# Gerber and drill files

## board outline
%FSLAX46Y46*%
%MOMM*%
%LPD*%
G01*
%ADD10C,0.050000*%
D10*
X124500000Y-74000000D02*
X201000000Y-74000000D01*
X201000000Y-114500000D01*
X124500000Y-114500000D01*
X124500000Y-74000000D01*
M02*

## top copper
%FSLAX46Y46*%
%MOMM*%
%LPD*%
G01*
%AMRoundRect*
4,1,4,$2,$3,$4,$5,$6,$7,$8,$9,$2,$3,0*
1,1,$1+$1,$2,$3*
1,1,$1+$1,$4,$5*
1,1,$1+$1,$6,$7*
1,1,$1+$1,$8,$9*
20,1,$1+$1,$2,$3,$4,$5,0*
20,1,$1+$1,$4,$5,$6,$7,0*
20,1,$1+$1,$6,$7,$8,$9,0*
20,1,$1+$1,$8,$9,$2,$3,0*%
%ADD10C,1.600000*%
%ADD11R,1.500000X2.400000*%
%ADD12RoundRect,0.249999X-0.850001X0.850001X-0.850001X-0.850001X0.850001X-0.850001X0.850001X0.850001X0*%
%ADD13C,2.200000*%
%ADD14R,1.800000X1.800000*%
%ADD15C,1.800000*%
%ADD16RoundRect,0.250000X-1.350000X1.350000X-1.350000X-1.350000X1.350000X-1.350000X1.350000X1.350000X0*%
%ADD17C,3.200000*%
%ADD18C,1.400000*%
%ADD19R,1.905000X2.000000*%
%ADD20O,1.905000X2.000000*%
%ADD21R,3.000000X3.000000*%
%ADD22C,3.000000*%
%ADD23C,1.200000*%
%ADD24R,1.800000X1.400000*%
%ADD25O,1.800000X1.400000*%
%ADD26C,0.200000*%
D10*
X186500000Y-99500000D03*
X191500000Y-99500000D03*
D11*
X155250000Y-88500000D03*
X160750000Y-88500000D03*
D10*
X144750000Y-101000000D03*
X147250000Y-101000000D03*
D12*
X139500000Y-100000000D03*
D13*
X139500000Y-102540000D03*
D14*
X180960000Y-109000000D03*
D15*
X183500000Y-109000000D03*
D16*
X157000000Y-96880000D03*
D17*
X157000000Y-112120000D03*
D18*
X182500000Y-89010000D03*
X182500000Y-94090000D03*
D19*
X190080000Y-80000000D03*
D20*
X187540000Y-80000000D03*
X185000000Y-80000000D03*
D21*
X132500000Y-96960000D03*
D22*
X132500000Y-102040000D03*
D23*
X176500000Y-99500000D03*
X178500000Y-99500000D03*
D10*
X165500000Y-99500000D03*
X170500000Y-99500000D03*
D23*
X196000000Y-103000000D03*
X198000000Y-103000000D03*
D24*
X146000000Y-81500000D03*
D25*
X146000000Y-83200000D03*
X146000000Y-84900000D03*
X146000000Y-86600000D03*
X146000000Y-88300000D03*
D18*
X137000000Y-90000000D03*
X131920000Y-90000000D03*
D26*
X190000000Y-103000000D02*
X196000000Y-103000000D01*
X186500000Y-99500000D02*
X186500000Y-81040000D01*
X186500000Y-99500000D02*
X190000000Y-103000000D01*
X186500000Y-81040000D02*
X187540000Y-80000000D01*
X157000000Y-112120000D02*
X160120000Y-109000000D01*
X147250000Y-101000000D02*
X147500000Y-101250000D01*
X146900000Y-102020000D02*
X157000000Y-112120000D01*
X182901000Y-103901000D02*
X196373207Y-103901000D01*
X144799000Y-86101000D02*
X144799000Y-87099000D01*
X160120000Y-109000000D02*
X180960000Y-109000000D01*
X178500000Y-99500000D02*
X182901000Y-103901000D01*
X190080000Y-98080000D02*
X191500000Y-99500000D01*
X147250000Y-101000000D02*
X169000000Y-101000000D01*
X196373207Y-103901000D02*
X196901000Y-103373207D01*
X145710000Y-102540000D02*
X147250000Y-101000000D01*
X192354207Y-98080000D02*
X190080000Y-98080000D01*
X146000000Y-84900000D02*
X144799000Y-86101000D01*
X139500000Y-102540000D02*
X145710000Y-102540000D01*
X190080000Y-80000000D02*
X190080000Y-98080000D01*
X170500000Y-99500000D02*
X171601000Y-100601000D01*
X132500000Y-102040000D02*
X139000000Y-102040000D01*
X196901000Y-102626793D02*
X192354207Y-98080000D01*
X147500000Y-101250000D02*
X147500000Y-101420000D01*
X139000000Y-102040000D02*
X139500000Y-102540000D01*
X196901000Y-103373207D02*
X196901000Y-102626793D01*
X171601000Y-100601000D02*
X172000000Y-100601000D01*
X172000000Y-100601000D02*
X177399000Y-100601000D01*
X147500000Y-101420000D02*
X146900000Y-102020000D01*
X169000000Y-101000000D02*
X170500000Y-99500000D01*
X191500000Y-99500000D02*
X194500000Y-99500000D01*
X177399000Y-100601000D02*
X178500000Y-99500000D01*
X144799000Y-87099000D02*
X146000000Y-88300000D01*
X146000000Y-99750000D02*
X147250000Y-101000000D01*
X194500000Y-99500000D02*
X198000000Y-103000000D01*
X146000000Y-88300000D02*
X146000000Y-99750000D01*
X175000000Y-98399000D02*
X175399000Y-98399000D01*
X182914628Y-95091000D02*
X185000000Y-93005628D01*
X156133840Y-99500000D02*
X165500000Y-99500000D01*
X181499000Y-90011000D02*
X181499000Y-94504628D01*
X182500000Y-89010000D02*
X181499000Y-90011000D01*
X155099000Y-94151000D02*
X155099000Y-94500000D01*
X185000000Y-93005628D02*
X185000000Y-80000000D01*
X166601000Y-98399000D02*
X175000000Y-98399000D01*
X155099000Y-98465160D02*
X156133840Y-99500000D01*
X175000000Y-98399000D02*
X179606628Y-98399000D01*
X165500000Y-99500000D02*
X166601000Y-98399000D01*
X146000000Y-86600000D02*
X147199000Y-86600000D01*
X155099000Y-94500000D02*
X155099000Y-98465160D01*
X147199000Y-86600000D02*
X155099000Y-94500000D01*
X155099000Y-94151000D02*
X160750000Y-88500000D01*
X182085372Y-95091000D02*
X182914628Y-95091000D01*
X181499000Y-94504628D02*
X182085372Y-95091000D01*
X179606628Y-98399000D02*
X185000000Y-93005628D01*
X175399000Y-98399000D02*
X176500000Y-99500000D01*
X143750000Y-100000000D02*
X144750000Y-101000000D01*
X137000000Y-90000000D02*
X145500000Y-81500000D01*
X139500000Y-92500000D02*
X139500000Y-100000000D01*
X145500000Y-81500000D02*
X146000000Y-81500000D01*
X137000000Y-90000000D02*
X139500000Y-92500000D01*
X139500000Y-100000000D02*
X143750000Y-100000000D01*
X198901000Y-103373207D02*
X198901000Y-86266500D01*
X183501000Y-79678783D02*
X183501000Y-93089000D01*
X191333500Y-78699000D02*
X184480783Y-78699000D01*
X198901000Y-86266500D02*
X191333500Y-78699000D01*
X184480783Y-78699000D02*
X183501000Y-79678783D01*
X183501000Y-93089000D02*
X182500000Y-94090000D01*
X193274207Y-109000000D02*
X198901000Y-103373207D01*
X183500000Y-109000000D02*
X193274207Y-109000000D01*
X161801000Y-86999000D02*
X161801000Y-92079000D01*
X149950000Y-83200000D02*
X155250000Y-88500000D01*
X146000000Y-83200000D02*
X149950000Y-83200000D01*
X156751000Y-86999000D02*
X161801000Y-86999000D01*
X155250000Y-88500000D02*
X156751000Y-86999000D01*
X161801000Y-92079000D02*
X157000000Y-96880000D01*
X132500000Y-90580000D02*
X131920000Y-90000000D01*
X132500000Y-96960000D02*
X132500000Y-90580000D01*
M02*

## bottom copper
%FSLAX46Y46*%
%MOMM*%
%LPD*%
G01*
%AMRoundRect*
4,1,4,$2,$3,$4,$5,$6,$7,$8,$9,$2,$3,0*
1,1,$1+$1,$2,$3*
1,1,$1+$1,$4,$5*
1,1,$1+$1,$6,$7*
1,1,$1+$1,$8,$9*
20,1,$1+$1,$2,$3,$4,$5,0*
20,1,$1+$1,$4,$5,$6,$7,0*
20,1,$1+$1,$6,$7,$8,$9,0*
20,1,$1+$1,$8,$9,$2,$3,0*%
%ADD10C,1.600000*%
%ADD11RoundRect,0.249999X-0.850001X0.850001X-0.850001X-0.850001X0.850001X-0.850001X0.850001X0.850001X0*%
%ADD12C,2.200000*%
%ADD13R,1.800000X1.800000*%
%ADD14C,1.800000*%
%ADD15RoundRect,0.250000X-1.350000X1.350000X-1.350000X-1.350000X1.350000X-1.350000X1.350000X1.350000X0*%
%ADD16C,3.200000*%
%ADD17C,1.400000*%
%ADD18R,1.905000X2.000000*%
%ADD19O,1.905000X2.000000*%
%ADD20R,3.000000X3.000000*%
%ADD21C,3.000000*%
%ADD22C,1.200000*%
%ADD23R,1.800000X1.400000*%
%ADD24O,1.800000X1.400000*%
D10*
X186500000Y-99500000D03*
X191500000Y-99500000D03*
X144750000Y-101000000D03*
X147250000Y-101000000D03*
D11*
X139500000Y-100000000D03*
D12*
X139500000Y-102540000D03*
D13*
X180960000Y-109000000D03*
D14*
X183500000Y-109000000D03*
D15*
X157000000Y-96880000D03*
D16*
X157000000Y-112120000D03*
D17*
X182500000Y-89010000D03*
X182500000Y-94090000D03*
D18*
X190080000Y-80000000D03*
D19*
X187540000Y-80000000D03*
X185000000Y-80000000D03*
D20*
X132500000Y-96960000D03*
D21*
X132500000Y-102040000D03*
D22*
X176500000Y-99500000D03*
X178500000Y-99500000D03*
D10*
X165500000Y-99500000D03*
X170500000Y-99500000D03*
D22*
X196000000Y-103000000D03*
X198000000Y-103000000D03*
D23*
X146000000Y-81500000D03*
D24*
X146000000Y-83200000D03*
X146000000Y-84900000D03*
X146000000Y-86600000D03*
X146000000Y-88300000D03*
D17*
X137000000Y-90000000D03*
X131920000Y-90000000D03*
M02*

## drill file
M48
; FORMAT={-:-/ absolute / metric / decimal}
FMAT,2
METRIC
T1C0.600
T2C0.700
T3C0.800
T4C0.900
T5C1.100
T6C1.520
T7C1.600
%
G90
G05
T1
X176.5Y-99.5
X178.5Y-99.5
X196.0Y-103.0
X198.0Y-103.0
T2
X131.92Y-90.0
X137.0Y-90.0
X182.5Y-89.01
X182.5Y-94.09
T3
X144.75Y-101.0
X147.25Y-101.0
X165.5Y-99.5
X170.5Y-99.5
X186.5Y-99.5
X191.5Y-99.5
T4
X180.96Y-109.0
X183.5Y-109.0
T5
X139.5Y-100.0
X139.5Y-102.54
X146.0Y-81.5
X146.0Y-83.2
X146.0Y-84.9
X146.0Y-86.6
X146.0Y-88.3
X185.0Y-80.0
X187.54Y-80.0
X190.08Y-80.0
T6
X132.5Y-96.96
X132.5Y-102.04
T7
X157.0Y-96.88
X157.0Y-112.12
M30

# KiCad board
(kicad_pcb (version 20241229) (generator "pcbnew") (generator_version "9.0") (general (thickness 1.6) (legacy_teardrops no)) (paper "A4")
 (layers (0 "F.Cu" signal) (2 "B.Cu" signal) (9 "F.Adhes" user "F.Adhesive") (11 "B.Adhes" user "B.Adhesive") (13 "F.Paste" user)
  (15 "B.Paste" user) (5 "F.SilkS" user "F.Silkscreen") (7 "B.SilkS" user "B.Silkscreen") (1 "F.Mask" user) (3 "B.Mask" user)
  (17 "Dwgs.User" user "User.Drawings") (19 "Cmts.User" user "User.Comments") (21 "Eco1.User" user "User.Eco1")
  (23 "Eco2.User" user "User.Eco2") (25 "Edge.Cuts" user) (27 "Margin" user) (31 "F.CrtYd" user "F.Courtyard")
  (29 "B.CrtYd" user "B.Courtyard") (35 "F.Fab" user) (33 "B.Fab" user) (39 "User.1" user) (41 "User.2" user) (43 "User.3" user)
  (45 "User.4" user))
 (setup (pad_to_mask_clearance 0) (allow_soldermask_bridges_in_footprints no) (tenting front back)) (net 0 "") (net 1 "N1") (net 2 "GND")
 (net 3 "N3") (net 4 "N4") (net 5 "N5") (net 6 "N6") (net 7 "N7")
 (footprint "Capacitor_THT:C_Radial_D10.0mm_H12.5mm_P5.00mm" (layer "F.Cu") (at 186.5 99.5)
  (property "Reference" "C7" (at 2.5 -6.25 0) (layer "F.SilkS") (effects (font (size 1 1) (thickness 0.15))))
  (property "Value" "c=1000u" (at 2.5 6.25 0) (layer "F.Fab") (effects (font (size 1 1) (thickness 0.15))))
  (pad "1" thru_hole circle (at 0 0) (size 1.6 1.6) (drill 0.8) (layers "*.Cu" "*.Mask") (remove_unused_layers no) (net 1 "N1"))
  (pad "2" thru_hole circle (at 5 0) (size 1.6 1.6) (drill 0.8) (layers "*.Cu" "*.Mask") (remove_unused_layers no) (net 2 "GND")))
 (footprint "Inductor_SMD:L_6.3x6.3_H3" (layer "F.Cu") (at 158 88.5)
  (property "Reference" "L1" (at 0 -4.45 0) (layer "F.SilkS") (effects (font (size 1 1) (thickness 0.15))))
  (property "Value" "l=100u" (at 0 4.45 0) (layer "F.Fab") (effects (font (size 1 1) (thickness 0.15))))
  (pad "1" smd rect (at -2.75 0) (size 1.5 2.4) (layers "F.Cu" "F.Mask" "F.Paste") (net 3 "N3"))
  (pad "2" smd rect (at 2.75 0) (size 1.5 2.4) (layers "F.Cu" "F.Mask" "F.Paste") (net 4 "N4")))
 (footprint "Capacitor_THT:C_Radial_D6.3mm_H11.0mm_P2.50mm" (layer "F.Cu") (at 144.75 101)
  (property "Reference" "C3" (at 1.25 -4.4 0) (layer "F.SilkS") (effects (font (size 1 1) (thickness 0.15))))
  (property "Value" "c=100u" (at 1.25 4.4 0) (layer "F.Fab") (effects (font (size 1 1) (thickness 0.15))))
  (pad "1" thru_hole circle (at 0 0) (size 1.6 1.6) (drill 0.8) (layers "*.Cu" "*.Mask") (remove_unused_layers no) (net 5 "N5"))
  (pad "2" thru_hole circle (at 2.5 0) (size 1.6 1.6) (drill 0.8) (layers "*.Cu" "*.Mask") (remove_unused_layers no) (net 2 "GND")))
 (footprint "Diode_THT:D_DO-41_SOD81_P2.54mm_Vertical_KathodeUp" (layer "F.Cu") (at 139.5 100 -90)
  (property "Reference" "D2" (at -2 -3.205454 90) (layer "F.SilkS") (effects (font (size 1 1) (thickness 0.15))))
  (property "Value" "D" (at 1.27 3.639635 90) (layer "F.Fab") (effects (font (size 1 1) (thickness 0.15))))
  (pad "1" thru_hole roundrect (at 0 0 270) (size 2.2 2.2) (drill 1.1) (layers "*.Cu" "*.Mask") (remove_unused_layers no)
   (roundrect_rratio 0.113636) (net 5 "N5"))
  (pad "2" thru_hole circle (at 2.54 0 270) (size 2.2 2.2) (drill 1.1) (layers "*.Cu" "*.Mask") (remove_unused_layers no) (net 2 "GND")))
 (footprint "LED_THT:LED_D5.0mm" (layer "F.Cu") (at 180.96 109)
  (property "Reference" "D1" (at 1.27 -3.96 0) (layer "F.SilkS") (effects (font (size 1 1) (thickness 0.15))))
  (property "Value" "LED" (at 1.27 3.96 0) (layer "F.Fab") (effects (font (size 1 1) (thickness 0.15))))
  (pad "1" thru_hole rect (at 0 0) (size 1.8 1.8) (drill 0.9) (layers "*.Cu" "*.Mask") (remove_unused_layers no) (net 2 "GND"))
  (pad "2" thru_hole circle (at 2.54 0) (size 1.8 1.8) (drill 0.9) (layers "*.Cu" "*.Mask") (remove_unused_layers no) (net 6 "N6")))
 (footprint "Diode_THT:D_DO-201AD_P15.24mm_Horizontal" (layer "F.Cu") (at 157 96.88 -90)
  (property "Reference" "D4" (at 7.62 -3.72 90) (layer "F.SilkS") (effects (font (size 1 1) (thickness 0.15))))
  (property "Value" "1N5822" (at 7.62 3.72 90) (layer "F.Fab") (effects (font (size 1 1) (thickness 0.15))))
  (pad "1" thru_hole roundrect (at 0 0 270) (size 3.2 3.2) (drill 1.6) (layers "*.Cu" "*.Mask") (remove_unused_layers no)
   (roundrect_rratio 0.078125) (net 3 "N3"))
  (pad "2" thru_hole circle (at 15.24 0 270) (size 3.2 3.2) (drill 1.6) (layers "*.Cu" "*.Mask") (remove_unused_layers no) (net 2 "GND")))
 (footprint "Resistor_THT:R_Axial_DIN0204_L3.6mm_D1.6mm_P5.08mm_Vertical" (layer "F.Cu") (at 182.5 89.01 -90)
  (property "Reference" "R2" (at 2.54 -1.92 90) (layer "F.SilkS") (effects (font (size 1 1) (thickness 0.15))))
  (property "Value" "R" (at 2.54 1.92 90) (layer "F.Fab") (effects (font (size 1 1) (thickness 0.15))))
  (pad "1" thru_hole circle (at 0 0 270) (size 1.4 1.4) (drill 0.7) (layers "*.Cu" "*.Mask") (remove_unused_layers no) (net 4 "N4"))
  (pad "2" thru_hole circle (at 5.08 0 270) (size 1.4 1.4) (drill 0.7) (layers "*.Cu" "*.Mask") (remove_unused_layers no) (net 6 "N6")))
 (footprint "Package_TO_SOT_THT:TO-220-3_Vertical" (layer "F.Cu") (at 190.08 80 180)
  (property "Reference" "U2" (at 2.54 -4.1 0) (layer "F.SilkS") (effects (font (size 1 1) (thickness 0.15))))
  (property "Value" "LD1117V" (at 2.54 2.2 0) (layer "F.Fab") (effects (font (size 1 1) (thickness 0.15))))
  (pad "1" thru_hole rect (at 0 0 180) (size 1.905 2) (drill 1.1) (layers "*.Cu" "*.Mask") (remove_unused_layers no) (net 2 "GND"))
  (pad "2" thru_hole oval (at 2.54 0 180) (size 1.905 2) (drill 1.1) (layers "*.Cu" "*.Mask") (remove_unused_layers no) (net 1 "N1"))
  (pad "3" thru_hole oval (at 5.08 0 180) (size 1.905 2) (drill 1.1) (layers "*.Cu" "*.Mask") (remove_unused_layers no) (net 4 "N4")))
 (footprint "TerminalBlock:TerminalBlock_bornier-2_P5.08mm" (layer "F.Cu") (at 132.5 96.96 -90)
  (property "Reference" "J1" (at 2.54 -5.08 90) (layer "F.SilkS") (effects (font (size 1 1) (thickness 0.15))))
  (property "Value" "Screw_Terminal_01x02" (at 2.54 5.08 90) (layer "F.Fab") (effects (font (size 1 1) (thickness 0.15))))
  (pad "1" thru_hole rect (at 0 0 270) (size 3 3) (drill 1.52) (layers "*.Cu" "*.Mask") (remove_unused_layers no) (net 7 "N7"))
  (pad "2" thru_hole circle (at 5.08 0 270) (size 3 3) (drill 1.52) (layers "*.Cu" "*.Mask") (remove_unused_layers no) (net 2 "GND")))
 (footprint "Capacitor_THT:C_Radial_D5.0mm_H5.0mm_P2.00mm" (layer "F.Cu") (at 176.5 99.5)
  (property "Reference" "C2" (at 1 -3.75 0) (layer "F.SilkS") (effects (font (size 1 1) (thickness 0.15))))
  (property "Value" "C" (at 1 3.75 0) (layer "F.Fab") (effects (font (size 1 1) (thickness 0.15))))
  (pad "1" thru_hole circle (at 0 0) (size 1.2 1.2) (drill 0.6) (layers "*.Cu" "*.Mask") (remove_unused_layers no) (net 4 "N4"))
  (pad "2" thru_hole circle (at 2 0) (size 1.2 1.2) (drill 0.6) (layers "*.Cu" "*.Mask") (remove_unused_layers no) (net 2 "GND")))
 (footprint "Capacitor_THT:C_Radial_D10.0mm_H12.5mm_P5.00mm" (layer "F.Cu") (at 165.5 99.5)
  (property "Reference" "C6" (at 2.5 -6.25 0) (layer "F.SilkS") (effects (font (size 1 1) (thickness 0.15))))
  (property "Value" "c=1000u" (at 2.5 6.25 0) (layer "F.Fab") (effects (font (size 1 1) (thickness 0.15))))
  (pad "1" thru_hole circle (at 0 0) (size 1.6 1.6) (drill 0.8) (layers "*.Cu" "*.Mask") (remove_unused_layers no) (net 4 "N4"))
  (pad "2" thru_hole circle (at 5 0) (size 1.6 1.6) (drill 0.8) (layers "*.Cu" "*.Mask") (remove_unused_layers no) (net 2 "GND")))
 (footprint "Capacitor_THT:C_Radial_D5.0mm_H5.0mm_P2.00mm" (layer "F.Cu") (at 196 103)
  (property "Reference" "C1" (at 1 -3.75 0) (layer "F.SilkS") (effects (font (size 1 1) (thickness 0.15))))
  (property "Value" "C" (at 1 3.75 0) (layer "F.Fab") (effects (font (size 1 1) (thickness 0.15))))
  (pad "1" thru_hole circle (at 0 0) (size 1.2 1.2) (drill 0.6) (layers "*.Cu" "*.Mask") (remove_unused_layers no) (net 1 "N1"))
  (pad "2" thru_hole circle (at 2 0) (size 1.2 1.2) (drill 0.6) (layers "*.Cu" "*.Mask") (remove_unused_layers no) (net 2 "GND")))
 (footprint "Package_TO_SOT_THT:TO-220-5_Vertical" (layer "F.Cu") (at 146 81.5 -90)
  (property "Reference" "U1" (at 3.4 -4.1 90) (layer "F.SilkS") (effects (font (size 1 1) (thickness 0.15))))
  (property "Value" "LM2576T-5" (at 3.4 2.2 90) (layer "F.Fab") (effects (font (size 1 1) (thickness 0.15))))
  (pad "1" thru_hole rect (at 0 0 270) (size 1.4 1.8) (drill 1.1) (layers "*.Cu" "*.Mask") (remove_unused_layers no) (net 5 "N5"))
  (pad "2" thru_hole oval (at 1.7 0 270) (size 1.4 1.8) (drill 1.1) (layers "*.Cu" "*.Mask") (remove_unused_layers no) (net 3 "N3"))
  (pad "3" thru_hole oval (at 3.4 0 270) (size 1.4 1.8) (drill 1.1) (layers "*.Cu" "*.Mask") (remove_unused_layers no) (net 2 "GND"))
  (pad "4" thru_hole oval (at 5.1 0 270) (size 1.4 1.8) (drill 1.1) (layers "*.Cu" "*.Mask") (remove_unused_layers no) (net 4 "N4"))
  (pad "5" thru_hole oval (at 6.8 0 270) (size 1.4 1.8) (drill 1.1) (layers "*.Cu" "*.Mask") (remove_unused_layers no) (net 2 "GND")))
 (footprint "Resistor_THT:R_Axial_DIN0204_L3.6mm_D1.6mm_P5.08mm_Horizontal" (layer "F.Cu") (at 137 90 180)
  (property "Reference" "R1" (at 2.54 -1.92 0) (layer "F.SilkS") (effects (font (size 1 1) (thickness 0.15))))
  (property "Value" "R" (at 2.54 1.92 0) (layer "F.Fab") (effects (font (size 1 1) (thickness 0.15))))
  (pad "1" thru_hole circle (at 0 0 180) (size 1.4 1.4) (drill 0.7) (layers "*.Cu" "*.Mask") (remove_unused_layers no) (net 5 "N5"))
  (pad "2" thru_hole circle (at 5.08 0 180) (size 1.4 1.4) (drill 0.7) (layers "*.Cu" "*.Mask") (remove_unused_layers no) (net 7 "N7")))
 (gr_rect (start 124.5 74) (end 201 114.5) (stroke (width 0.05) (type default)) (fill no) (layer "Edge.Cuts"))
 (segment (start 190 103) (end 196 103) (width 0.2) (layer "F.Cu") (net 1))
 (segment (start 186.5 99.5) (end 186.5 81.04) (width 0.2) (layer "F.Cu") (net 1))
 (segment (start 186.5 99.5) (end 190 103) (width 0.2) (layer "F.Cu") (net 1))
 (segment (start 186.5 81.04) (end 187.54 80) (width 0.2) (layer "F.Cu") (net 1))
 (segment (start 157 112.12) (end 160.12 109) (width 0.2) (layer "F.Cu") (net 2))
 (segment (start 147.25 101) (end 147.5 101.25) (width 0.2) (layer "F.Cu") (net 2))
 (segment (start 146.9 102.02) (end 157 112.12) (width 0.2) (layer "F.Cu") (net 2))
 (segment (start 182.901 103.901) (end 196.373207 103.901) (width 0.2) (layer "F.Cu") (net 2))
 (segment (start 144.799 86.101) (end 144.799 87.099) (width 0.2) (layer "F.Cu") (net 2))
 (segment (start 160.12 109) (end 180.96 109) (width 0.2) (layer "F.Cu") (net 2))
 (segment (start 178.5 99.5) (end 182.901 103.901) (width 0.2) (layer "F.Cu") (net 2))
 (segment (start 190.08 98.08) (end 191.5 99.5) (width 0.2) (layer "F.Cu") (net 2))
 (segment (start 147.25 101) (end 169 101) (width 0.2) (layer "F.Cu") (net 2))
 (segment (start 196.373207 103.901) (end 196.901 103.373207) (width 0.2) (layer "F.Cu") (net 2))
 (segment (start 145.71 102.54) (end 147.25 101) (width 0.2) (layer "F.Cu") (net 2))
 (segment (start 192.354207 98.08) (end 190.08 98.08) (width 0.2) (layer "F.Cu") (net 2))
 (segment (start 146 84.9) (end 144.799 86.101) (width 0.2) (layer "F.Cu") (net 2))
 (segment (start 139.5 102.54) (end 145.71 102.54) (width 0.2) (layer "F.Cu") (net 2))
 (segment (start 190.08 80) (end 190.08 98.08) (width 0.2) (layer "F.Cu") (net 2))
 (segment (start 170.5 99.5) (end 171.601 100.601) (width 0.2) (layer "F.Cu") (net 2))
 (segment (start 132.5 102.04) (end 139 102.04) (width 0.2) (layer "F.Cu") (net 2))
 (segment (start 196.901 102.626793) (end 192.354207 98.08) (width 0.2) (layer "F.Cu") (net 2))
 (segment (start 147.5 101.25) (end 147.5 101.42) (width 0.2) (layer "F.Cu") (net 2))
 (segment (start 139 102.04) (end 139.5 102.54) (width 0.2) (layer "F.Cu") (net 2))
 (segment (start 196.901 103.373207) (end 196.901 102.626793) (width 0.2) (layer "F.Cu") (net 2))
 (segment (start 171.601 100.601) (end 172 100.601) (width 0.2) (layer "F.Cu") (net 2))
 (segment (start 172 100.601) (end 177.399 100.601) (width 0.2) (layer "F.Cu") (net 2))
 (segment (start 147.5 101.42) (end 146.9 102.02) (width 0.2) (layer "F.Cu") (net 2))
 (segment (start 169 101) (end 170.5 99.5) (width 0.2) (layer "F.Cu") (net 2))
 (segment (start 191.5 99.5) (end 194.5 99.5) (width 0.2) (layer "F.Cu") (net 2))
 (segment (start 177.399 100.601) (end 178.5 99.5) (width 0.2) (layer "F.Cu") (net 2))
 (segment (start 144.799 87.099) (end 146 88.3) (width 0.2) (layer "F.Cu") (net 2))
 (segment (start 146 99.75) (end 147.25 101) (width 0.2) (layer "F.Cu") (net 2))
 (segment (start 194.5 99.5) (end 198 103) (width 0.2) (layer "F.Cu") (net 2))
 (segment (start 146 88.3) (end 146 99.75) (width 0.2) (layer "F.Cu") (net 2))
 (segment (start 175 98.399) (end 175.399 98.399) (width 0.2) (layer "F.Cu") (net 4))
 (segment (start 182.914628 95.091) (end 185 93.005628) (width 0.2) (layer "F.Cu") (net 4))
 (segment (start 156.13384 99.5) (end 165.5 99.5) (width 0.2) (layer "F.Cu") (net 4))
 (segment (start 181.499 90.011) (end 181.499 94.504628) (width 0.2) (layer "F.Cu") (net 4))
 (segment (start 182.5 89.01) (end 181.499 90.011) (width 0.2) (layer "F.Cu") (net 4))
 (segment (start 155.099 94.151) (end 155.099 94.5) (width 0.2) (layer "F.Cu") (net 4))
 (segment (start 185 93.005628) (end 185 80) (width 0.2) (layer "F.Cu") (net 4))
 (segment (start 166.601 98.399) (end 175 98.399) (width 0.2) (layer "F.Cu") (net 4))
 (segment (start 155.099 98.46516) (end 156.13384 99.5) (width 0.2) (layer "F.Cu") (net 4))
 (segment (start 175 98.399) (end 179.606628 98.399) (width 0.2) (layer "F.Cu") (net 4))
 (segment (start 165.5 99.5) (end 166.601 98.399) (width 0.2) (layer "F.Cu") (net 4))
 (segment (start 146 86.6) (end 147.199 86.6) (width 0.2) (layer "F.Cu") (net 4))
 (segment (start 155.099 94.5) (end 155.099 98.46516) (width 0.2) (layer "F.Cu") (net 4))
 (segment (start 147.199 86.6) (end 155.099 94.5) (width 0.2) (layer "F.Cu") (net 4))
 (segment (start 155.099 94.151) (end 160.75 88.5) (width 0.2) (layer "F.Cu") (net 4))
 (segment (start 182.085372 95.091) (end 182.914628 95.091) (width 0.2) (layer "F.Cu") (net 4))
 (segment (start 181.499 94.504628) (end 182.085372 95.091) (width 0.2) (layer "F.Cu") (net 4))
 (segment (start 179.606628 98.399) (end 185 93.005628) (width 0.2) (layer "F.Cu") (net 4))
 (segment (start 175.399 98.399) (end 176.5 99.5) (width 0.2) (layer "F.Cu") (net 4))
 (segment (start 143.75 100) (end 144.75 101) (width 0.2) (layer "F.Cu") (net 5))
 (segment (start 137 90) (end 145.5 81.5) (width 0.2) (layer "F.Cu") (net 5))
 (segment (start 139.5 92.5) (end 139.5 100) (width 0.2) (layer "F.Cu") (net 5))
 (segment (start 145.5 81.5) (end 146 81.5) (width 0.2) (layer "F.Cu") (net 5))
 (segment (start 137 90) (end 139.5 92.5) (width 0.2) (layer "F.Cu") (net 5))
 (segment (start 139.5 100) (end 143.75 100) (width 0.2) (layer "F.Cu") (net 5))
 (segment (start 198.901 103.373207) (end 198.901 86.2665) (width 0.2) (layer "F.Cu") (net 6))
 (segment (start 183.501 79.678783) (end 183.501 93.089) (width 0.2) (layer "F.Cu") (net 6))
 (segment (start 191.3335 78.699) (end 184.480783 78.699) (width 0.2) (layer "F.Cu") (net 6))
 (segment (start 198.901 86.2665) (end 191.3335 78.699) (width 0.2) (layer "F.Cu") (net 6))
 (segment (start 184.480783 78.699) (end 183.501 79.678783) (width 0.2) (layer "F.Cu") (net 6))
 (segment (start 183.501 93.089) (end 182.5 94.09) (width 0.2) (layer "F.Cu") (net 6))
 (segment (start 193.274207 109) (end 198.901 103.373207) (width 0.2) (layer "F.Cu") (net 6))
 (segment (start 183.5 109) (end 193.274207 109) (width 0.2) (layer "F.Cu") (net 6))
 (segment (start 161.801 86.999) (end 161.801 92.079) (width 0.2) (layer "F.Cu") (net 3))
 (segment (start 149.95 83.2) (end 155.25 88.5) (width 0.2) (layer "F.Cu") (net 3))
 (segment (start 146 83.2) (end 149.95 83.2) (width 0.2) (layer "F.Cu") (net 3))
 (segment (start 156.751 86.999) (end 161.801 86.999) (width 0.2) (layer "F.Cu") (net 3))
 (segment (start 155.25 88.5) (end 156.751 86.999) (width 0.2) (layer "F.Cu") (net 3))
 (segment (start 161.801 92.079) (end 157 96.88) (width 0.2) (layer "F.Cu") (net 3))
 (segment (start 132.5 90.58) (end 131.92 90) (width 0.2) (layer "F.Cu") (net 7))
 (segment (start 132.5 96.96) (end 132.5 90.58) (width 0.2) (layer "F.Cu") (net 7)))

